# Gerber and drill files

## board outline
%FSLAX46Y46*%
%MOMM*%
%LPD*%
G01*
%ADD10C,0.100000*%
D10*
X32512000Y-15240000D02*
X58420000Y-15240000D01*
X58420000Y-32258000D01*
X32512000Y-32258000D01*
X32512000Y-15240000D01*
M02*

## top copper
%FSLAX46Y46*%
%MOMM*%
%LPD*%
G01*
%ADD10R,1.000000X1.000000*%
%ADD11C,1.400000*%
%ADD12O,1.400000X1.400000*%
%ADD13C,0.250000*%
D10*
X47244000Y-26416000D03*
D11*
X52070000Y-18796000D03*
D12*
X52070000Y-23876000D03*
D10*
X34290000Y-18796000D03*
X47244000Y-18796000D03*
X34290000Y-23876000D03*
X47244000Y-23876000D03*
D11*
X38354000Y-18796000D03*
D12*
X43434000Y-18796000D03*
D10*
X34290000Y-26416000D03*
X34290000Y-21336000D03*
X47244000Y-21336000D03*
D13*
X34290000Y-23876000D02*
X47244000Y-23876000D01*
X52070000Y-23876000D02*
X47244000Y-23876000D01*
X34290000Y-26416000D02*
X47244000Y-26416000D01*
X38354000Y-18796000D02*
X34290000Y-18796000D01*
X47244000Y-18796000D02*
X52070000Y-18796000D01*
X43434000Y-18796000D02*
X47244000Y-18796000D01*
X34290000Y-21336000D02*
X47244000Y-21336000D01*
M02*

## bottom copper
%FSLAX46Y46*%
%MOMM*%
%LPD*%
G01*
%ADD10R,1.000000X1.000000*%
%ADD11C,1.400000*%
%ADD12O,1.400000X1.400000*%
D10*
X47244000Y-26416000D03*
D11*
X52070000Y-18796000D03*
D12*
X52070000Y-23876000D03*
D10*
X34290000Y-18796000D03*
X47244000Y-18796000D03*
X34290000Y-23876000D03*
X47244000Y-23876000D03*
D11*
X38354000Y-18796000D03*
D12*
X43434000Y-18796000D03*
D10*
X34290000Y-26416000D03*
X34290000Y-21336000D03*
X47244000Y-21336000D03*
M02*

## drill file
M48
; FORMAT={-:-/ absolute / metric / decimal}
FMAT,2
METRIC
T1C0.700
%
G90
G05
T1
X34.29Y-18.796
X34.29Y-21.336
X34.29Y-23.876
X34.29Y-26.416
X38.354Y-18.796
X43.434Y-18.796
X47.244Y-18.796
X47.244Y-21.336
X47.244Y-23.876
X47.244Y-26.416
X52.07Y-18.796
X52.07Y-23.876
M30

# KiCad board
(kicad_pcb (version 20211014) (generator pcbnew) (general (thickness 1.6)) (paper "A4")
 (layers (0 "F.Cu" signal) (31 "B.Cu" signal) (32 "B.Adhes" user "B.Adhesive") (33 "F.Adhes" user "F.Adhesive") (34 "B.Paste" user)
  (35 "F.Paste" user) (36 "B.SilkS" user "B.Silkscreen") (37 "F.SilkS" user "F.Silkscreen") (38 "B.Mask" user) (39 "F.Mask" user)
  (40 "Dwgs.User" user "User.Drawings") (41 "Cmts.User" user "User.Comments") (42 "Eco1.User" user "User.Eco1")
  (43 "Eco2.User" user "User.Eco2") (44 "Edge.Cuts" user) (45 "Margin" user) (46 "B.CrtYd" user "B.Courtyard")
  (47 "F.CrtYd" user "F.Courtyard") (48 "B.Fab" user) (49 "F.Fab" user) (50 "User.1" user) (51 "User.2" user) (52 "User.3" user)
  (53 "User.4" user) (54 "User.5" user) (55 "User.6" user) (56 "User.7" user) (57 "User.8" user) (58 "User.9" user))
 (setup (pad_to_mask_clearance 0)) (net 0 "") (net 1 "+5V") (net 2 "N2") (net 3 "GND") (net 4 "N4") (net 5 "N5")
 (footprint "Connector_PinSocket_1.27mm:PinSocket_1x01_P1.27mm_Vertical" (layer "F.Cu") (at 47.244 26.416 90)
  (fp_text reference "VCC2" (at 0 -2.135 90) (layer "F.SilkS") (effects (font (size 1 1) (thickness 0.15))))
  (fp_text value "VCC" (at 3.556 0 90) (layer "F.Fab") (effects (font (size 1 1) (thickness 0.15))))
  (pad "1" thru_hole rect (at 0 0 90) (size 1 1) (drill 0.7) (layers *.Cu *.Mask) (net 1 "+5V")))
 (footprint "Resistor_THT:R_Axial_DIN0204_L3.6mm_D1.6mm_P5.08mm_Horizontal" (layer "F.Cu") (at 52.07 18.796 -90)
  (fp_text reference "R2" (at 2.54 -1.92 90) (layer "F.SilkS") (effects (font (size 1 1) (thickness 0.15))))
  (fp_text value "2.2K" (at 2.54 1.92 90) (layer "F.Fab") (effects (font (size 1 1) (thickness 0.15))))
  (pad "1" thru_hole circle (at 0 0 270) (size 1.4 1.4) (drill 0.7) (layers *.Cu *.Mask) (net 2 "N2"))
  (pad "2" thru_hole oval (at 5.08 0 270) (size 1.4 1.4) (drill 0.7) (layers *.Cu *.Mask) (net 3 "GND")))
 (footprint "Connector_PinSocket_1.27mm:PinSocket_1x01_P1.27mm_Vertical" (layer "F.Cu") (at 34.29 18.796 90)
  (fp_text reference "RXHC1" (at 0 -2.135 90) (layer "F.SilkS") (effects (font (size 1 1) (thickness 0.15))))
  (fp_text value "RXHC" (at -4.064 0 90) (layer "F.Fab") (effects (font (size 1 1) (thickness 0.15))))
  (pad "1" thru_hole rect (at 0 0 90) (size 1 1) (drill 0.7) (layers *.Cu *.Mask) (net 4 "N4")))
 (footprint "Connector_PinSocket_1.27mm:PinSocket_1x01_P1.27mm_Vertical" (layer "F.Cu") (at 47.244 18.796 90)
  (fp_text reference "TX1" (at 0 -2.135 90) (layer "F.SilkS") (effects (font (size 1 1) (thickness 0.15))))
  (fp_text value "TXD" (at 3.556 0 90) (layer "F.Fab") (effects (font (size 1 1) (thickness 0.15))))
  (pad "1" thru_hole rect (at 0 0 90) (size 1 1) (drill 0.7) (layers *.Cu *.Mask) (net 2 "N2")))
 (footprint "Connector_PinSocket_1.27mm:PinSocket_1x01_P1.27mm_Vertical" (layer "F.Cu") (at 34.29 23.876 90)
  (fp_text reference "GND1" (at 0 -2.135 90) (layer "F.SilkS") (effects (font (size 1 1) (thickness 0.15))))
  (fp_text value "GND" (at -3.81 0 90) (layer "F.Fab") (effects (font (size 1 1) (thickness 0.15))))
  (pad "1" thru_hole rect (at 0 0 90) (size 1 1) (drill 0.7) (layers *.Cu *.Mask) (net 3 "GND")))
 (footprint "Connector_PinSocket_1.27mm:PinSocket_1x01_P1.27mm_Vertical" (layer "F.Cu") (at 47.244 23.876 90)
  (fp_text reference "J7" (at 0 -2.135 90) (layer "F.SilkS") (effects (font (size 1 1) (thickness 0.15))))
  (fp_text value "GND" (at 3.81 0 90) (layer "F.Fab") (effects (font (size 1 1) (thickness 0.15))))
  (pad "1" thru_hole rect (at 0 0 90) (size 1 1) (drill 0.7) (layers *.Cu *.Mask) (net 3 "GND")))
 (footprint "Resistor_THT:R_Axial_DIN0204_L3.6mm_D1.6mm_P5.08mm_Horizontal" (layer "F.Cu") (at 38.354 18.796)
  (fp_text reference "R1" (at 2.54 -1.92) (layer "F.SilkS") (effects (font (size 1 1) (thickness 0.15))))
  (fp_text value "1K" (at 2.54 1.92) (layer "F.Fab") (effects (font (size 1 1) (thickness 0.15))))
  (pad "1" thru_hole circle (at 0 0) (size 1.4 1.4) (drill 0.7) (layers *.Cu *.Mask) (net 4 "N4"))
  (pad "2" thru_hole oval (at 5.08 0) (size 1.4 1.4) (drill 0.7) (layers *.Cu *.Mask) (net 2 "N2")))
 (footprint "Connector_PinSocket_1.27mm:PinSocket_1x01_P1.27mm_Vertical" (layer "F.Cu") (at 34.29 26.416 90)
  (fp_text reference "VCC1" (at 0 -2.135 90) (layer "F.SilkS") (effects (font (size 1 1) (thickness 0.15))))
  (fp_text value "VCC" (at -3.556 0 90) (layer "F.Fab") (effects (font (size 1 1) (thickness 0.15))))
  (pad "1" thru_hole rect (at 0 0 90) (size 1 1) (drill 0.7) (layers *.Cu *.Mask) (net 1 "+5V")))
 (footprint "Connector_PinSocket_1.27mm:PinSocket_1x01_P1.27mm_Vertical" (layer "F.Cu") (at 34.29 21.336 90)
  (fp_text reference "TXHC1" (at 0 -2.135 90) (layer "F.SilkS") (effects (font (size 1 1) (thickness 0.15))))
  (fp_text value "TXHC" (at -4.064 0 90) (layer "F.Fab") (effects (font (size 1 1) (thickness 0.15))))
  (pad "1" thru_hole rect (at 0 0 90) (size 1 1) (drill 0.7) (layers *.Cu *.Mask) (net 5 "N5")))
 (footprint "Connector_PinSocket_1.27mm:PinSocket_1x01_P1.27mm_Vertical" (layer "F.Cu") (at 47.244 21.336 90)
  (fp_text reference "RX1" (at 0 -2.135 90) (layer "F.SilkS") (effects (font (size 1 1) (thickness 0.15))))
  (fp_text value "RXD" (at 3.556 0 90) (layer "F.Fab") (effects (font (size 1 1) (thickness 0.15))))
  (pad "1" thru_hole rect (at 0 0 90) (size 1 1) (drill 0.7) (layers *.Cu *.Mask) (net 5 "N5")))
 (gr_rect (start 32.512 15.24) (end 58.42 32.258) (layer "Edge.Cuts") (width 0.1) (fill none))
 (segment (start 34.29 23.876) (end 47.244 23.876) (width 0.25) (layer "F.Cu") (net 3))
 (segment (start 52.07 23.876) (end 47.244 23.876) (width 0.25) (layer "F.Cu") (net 3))
 (segment (start 34.29 26.416) (end 47.244 26.416) (width 0.25) (layer "F.Cu") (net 1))
 (segment (start 38.354 18.796) (end 34.29 18.796) (width 0.25) (layer "F.Cu") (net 4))
 (segment (start 47.244 18.796) (end 52.07 18.796) (width 0.25) (layer "F.Cu") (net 2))
 (segment (start 43.434 18.796) (end 47.244 18.796) (width 0.25) (layer "F.Cu") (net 2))
 (segment (start 34.29 21.336) (end 47.244 21.336) (width 0.25) (layer "F.Cu") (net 5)))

